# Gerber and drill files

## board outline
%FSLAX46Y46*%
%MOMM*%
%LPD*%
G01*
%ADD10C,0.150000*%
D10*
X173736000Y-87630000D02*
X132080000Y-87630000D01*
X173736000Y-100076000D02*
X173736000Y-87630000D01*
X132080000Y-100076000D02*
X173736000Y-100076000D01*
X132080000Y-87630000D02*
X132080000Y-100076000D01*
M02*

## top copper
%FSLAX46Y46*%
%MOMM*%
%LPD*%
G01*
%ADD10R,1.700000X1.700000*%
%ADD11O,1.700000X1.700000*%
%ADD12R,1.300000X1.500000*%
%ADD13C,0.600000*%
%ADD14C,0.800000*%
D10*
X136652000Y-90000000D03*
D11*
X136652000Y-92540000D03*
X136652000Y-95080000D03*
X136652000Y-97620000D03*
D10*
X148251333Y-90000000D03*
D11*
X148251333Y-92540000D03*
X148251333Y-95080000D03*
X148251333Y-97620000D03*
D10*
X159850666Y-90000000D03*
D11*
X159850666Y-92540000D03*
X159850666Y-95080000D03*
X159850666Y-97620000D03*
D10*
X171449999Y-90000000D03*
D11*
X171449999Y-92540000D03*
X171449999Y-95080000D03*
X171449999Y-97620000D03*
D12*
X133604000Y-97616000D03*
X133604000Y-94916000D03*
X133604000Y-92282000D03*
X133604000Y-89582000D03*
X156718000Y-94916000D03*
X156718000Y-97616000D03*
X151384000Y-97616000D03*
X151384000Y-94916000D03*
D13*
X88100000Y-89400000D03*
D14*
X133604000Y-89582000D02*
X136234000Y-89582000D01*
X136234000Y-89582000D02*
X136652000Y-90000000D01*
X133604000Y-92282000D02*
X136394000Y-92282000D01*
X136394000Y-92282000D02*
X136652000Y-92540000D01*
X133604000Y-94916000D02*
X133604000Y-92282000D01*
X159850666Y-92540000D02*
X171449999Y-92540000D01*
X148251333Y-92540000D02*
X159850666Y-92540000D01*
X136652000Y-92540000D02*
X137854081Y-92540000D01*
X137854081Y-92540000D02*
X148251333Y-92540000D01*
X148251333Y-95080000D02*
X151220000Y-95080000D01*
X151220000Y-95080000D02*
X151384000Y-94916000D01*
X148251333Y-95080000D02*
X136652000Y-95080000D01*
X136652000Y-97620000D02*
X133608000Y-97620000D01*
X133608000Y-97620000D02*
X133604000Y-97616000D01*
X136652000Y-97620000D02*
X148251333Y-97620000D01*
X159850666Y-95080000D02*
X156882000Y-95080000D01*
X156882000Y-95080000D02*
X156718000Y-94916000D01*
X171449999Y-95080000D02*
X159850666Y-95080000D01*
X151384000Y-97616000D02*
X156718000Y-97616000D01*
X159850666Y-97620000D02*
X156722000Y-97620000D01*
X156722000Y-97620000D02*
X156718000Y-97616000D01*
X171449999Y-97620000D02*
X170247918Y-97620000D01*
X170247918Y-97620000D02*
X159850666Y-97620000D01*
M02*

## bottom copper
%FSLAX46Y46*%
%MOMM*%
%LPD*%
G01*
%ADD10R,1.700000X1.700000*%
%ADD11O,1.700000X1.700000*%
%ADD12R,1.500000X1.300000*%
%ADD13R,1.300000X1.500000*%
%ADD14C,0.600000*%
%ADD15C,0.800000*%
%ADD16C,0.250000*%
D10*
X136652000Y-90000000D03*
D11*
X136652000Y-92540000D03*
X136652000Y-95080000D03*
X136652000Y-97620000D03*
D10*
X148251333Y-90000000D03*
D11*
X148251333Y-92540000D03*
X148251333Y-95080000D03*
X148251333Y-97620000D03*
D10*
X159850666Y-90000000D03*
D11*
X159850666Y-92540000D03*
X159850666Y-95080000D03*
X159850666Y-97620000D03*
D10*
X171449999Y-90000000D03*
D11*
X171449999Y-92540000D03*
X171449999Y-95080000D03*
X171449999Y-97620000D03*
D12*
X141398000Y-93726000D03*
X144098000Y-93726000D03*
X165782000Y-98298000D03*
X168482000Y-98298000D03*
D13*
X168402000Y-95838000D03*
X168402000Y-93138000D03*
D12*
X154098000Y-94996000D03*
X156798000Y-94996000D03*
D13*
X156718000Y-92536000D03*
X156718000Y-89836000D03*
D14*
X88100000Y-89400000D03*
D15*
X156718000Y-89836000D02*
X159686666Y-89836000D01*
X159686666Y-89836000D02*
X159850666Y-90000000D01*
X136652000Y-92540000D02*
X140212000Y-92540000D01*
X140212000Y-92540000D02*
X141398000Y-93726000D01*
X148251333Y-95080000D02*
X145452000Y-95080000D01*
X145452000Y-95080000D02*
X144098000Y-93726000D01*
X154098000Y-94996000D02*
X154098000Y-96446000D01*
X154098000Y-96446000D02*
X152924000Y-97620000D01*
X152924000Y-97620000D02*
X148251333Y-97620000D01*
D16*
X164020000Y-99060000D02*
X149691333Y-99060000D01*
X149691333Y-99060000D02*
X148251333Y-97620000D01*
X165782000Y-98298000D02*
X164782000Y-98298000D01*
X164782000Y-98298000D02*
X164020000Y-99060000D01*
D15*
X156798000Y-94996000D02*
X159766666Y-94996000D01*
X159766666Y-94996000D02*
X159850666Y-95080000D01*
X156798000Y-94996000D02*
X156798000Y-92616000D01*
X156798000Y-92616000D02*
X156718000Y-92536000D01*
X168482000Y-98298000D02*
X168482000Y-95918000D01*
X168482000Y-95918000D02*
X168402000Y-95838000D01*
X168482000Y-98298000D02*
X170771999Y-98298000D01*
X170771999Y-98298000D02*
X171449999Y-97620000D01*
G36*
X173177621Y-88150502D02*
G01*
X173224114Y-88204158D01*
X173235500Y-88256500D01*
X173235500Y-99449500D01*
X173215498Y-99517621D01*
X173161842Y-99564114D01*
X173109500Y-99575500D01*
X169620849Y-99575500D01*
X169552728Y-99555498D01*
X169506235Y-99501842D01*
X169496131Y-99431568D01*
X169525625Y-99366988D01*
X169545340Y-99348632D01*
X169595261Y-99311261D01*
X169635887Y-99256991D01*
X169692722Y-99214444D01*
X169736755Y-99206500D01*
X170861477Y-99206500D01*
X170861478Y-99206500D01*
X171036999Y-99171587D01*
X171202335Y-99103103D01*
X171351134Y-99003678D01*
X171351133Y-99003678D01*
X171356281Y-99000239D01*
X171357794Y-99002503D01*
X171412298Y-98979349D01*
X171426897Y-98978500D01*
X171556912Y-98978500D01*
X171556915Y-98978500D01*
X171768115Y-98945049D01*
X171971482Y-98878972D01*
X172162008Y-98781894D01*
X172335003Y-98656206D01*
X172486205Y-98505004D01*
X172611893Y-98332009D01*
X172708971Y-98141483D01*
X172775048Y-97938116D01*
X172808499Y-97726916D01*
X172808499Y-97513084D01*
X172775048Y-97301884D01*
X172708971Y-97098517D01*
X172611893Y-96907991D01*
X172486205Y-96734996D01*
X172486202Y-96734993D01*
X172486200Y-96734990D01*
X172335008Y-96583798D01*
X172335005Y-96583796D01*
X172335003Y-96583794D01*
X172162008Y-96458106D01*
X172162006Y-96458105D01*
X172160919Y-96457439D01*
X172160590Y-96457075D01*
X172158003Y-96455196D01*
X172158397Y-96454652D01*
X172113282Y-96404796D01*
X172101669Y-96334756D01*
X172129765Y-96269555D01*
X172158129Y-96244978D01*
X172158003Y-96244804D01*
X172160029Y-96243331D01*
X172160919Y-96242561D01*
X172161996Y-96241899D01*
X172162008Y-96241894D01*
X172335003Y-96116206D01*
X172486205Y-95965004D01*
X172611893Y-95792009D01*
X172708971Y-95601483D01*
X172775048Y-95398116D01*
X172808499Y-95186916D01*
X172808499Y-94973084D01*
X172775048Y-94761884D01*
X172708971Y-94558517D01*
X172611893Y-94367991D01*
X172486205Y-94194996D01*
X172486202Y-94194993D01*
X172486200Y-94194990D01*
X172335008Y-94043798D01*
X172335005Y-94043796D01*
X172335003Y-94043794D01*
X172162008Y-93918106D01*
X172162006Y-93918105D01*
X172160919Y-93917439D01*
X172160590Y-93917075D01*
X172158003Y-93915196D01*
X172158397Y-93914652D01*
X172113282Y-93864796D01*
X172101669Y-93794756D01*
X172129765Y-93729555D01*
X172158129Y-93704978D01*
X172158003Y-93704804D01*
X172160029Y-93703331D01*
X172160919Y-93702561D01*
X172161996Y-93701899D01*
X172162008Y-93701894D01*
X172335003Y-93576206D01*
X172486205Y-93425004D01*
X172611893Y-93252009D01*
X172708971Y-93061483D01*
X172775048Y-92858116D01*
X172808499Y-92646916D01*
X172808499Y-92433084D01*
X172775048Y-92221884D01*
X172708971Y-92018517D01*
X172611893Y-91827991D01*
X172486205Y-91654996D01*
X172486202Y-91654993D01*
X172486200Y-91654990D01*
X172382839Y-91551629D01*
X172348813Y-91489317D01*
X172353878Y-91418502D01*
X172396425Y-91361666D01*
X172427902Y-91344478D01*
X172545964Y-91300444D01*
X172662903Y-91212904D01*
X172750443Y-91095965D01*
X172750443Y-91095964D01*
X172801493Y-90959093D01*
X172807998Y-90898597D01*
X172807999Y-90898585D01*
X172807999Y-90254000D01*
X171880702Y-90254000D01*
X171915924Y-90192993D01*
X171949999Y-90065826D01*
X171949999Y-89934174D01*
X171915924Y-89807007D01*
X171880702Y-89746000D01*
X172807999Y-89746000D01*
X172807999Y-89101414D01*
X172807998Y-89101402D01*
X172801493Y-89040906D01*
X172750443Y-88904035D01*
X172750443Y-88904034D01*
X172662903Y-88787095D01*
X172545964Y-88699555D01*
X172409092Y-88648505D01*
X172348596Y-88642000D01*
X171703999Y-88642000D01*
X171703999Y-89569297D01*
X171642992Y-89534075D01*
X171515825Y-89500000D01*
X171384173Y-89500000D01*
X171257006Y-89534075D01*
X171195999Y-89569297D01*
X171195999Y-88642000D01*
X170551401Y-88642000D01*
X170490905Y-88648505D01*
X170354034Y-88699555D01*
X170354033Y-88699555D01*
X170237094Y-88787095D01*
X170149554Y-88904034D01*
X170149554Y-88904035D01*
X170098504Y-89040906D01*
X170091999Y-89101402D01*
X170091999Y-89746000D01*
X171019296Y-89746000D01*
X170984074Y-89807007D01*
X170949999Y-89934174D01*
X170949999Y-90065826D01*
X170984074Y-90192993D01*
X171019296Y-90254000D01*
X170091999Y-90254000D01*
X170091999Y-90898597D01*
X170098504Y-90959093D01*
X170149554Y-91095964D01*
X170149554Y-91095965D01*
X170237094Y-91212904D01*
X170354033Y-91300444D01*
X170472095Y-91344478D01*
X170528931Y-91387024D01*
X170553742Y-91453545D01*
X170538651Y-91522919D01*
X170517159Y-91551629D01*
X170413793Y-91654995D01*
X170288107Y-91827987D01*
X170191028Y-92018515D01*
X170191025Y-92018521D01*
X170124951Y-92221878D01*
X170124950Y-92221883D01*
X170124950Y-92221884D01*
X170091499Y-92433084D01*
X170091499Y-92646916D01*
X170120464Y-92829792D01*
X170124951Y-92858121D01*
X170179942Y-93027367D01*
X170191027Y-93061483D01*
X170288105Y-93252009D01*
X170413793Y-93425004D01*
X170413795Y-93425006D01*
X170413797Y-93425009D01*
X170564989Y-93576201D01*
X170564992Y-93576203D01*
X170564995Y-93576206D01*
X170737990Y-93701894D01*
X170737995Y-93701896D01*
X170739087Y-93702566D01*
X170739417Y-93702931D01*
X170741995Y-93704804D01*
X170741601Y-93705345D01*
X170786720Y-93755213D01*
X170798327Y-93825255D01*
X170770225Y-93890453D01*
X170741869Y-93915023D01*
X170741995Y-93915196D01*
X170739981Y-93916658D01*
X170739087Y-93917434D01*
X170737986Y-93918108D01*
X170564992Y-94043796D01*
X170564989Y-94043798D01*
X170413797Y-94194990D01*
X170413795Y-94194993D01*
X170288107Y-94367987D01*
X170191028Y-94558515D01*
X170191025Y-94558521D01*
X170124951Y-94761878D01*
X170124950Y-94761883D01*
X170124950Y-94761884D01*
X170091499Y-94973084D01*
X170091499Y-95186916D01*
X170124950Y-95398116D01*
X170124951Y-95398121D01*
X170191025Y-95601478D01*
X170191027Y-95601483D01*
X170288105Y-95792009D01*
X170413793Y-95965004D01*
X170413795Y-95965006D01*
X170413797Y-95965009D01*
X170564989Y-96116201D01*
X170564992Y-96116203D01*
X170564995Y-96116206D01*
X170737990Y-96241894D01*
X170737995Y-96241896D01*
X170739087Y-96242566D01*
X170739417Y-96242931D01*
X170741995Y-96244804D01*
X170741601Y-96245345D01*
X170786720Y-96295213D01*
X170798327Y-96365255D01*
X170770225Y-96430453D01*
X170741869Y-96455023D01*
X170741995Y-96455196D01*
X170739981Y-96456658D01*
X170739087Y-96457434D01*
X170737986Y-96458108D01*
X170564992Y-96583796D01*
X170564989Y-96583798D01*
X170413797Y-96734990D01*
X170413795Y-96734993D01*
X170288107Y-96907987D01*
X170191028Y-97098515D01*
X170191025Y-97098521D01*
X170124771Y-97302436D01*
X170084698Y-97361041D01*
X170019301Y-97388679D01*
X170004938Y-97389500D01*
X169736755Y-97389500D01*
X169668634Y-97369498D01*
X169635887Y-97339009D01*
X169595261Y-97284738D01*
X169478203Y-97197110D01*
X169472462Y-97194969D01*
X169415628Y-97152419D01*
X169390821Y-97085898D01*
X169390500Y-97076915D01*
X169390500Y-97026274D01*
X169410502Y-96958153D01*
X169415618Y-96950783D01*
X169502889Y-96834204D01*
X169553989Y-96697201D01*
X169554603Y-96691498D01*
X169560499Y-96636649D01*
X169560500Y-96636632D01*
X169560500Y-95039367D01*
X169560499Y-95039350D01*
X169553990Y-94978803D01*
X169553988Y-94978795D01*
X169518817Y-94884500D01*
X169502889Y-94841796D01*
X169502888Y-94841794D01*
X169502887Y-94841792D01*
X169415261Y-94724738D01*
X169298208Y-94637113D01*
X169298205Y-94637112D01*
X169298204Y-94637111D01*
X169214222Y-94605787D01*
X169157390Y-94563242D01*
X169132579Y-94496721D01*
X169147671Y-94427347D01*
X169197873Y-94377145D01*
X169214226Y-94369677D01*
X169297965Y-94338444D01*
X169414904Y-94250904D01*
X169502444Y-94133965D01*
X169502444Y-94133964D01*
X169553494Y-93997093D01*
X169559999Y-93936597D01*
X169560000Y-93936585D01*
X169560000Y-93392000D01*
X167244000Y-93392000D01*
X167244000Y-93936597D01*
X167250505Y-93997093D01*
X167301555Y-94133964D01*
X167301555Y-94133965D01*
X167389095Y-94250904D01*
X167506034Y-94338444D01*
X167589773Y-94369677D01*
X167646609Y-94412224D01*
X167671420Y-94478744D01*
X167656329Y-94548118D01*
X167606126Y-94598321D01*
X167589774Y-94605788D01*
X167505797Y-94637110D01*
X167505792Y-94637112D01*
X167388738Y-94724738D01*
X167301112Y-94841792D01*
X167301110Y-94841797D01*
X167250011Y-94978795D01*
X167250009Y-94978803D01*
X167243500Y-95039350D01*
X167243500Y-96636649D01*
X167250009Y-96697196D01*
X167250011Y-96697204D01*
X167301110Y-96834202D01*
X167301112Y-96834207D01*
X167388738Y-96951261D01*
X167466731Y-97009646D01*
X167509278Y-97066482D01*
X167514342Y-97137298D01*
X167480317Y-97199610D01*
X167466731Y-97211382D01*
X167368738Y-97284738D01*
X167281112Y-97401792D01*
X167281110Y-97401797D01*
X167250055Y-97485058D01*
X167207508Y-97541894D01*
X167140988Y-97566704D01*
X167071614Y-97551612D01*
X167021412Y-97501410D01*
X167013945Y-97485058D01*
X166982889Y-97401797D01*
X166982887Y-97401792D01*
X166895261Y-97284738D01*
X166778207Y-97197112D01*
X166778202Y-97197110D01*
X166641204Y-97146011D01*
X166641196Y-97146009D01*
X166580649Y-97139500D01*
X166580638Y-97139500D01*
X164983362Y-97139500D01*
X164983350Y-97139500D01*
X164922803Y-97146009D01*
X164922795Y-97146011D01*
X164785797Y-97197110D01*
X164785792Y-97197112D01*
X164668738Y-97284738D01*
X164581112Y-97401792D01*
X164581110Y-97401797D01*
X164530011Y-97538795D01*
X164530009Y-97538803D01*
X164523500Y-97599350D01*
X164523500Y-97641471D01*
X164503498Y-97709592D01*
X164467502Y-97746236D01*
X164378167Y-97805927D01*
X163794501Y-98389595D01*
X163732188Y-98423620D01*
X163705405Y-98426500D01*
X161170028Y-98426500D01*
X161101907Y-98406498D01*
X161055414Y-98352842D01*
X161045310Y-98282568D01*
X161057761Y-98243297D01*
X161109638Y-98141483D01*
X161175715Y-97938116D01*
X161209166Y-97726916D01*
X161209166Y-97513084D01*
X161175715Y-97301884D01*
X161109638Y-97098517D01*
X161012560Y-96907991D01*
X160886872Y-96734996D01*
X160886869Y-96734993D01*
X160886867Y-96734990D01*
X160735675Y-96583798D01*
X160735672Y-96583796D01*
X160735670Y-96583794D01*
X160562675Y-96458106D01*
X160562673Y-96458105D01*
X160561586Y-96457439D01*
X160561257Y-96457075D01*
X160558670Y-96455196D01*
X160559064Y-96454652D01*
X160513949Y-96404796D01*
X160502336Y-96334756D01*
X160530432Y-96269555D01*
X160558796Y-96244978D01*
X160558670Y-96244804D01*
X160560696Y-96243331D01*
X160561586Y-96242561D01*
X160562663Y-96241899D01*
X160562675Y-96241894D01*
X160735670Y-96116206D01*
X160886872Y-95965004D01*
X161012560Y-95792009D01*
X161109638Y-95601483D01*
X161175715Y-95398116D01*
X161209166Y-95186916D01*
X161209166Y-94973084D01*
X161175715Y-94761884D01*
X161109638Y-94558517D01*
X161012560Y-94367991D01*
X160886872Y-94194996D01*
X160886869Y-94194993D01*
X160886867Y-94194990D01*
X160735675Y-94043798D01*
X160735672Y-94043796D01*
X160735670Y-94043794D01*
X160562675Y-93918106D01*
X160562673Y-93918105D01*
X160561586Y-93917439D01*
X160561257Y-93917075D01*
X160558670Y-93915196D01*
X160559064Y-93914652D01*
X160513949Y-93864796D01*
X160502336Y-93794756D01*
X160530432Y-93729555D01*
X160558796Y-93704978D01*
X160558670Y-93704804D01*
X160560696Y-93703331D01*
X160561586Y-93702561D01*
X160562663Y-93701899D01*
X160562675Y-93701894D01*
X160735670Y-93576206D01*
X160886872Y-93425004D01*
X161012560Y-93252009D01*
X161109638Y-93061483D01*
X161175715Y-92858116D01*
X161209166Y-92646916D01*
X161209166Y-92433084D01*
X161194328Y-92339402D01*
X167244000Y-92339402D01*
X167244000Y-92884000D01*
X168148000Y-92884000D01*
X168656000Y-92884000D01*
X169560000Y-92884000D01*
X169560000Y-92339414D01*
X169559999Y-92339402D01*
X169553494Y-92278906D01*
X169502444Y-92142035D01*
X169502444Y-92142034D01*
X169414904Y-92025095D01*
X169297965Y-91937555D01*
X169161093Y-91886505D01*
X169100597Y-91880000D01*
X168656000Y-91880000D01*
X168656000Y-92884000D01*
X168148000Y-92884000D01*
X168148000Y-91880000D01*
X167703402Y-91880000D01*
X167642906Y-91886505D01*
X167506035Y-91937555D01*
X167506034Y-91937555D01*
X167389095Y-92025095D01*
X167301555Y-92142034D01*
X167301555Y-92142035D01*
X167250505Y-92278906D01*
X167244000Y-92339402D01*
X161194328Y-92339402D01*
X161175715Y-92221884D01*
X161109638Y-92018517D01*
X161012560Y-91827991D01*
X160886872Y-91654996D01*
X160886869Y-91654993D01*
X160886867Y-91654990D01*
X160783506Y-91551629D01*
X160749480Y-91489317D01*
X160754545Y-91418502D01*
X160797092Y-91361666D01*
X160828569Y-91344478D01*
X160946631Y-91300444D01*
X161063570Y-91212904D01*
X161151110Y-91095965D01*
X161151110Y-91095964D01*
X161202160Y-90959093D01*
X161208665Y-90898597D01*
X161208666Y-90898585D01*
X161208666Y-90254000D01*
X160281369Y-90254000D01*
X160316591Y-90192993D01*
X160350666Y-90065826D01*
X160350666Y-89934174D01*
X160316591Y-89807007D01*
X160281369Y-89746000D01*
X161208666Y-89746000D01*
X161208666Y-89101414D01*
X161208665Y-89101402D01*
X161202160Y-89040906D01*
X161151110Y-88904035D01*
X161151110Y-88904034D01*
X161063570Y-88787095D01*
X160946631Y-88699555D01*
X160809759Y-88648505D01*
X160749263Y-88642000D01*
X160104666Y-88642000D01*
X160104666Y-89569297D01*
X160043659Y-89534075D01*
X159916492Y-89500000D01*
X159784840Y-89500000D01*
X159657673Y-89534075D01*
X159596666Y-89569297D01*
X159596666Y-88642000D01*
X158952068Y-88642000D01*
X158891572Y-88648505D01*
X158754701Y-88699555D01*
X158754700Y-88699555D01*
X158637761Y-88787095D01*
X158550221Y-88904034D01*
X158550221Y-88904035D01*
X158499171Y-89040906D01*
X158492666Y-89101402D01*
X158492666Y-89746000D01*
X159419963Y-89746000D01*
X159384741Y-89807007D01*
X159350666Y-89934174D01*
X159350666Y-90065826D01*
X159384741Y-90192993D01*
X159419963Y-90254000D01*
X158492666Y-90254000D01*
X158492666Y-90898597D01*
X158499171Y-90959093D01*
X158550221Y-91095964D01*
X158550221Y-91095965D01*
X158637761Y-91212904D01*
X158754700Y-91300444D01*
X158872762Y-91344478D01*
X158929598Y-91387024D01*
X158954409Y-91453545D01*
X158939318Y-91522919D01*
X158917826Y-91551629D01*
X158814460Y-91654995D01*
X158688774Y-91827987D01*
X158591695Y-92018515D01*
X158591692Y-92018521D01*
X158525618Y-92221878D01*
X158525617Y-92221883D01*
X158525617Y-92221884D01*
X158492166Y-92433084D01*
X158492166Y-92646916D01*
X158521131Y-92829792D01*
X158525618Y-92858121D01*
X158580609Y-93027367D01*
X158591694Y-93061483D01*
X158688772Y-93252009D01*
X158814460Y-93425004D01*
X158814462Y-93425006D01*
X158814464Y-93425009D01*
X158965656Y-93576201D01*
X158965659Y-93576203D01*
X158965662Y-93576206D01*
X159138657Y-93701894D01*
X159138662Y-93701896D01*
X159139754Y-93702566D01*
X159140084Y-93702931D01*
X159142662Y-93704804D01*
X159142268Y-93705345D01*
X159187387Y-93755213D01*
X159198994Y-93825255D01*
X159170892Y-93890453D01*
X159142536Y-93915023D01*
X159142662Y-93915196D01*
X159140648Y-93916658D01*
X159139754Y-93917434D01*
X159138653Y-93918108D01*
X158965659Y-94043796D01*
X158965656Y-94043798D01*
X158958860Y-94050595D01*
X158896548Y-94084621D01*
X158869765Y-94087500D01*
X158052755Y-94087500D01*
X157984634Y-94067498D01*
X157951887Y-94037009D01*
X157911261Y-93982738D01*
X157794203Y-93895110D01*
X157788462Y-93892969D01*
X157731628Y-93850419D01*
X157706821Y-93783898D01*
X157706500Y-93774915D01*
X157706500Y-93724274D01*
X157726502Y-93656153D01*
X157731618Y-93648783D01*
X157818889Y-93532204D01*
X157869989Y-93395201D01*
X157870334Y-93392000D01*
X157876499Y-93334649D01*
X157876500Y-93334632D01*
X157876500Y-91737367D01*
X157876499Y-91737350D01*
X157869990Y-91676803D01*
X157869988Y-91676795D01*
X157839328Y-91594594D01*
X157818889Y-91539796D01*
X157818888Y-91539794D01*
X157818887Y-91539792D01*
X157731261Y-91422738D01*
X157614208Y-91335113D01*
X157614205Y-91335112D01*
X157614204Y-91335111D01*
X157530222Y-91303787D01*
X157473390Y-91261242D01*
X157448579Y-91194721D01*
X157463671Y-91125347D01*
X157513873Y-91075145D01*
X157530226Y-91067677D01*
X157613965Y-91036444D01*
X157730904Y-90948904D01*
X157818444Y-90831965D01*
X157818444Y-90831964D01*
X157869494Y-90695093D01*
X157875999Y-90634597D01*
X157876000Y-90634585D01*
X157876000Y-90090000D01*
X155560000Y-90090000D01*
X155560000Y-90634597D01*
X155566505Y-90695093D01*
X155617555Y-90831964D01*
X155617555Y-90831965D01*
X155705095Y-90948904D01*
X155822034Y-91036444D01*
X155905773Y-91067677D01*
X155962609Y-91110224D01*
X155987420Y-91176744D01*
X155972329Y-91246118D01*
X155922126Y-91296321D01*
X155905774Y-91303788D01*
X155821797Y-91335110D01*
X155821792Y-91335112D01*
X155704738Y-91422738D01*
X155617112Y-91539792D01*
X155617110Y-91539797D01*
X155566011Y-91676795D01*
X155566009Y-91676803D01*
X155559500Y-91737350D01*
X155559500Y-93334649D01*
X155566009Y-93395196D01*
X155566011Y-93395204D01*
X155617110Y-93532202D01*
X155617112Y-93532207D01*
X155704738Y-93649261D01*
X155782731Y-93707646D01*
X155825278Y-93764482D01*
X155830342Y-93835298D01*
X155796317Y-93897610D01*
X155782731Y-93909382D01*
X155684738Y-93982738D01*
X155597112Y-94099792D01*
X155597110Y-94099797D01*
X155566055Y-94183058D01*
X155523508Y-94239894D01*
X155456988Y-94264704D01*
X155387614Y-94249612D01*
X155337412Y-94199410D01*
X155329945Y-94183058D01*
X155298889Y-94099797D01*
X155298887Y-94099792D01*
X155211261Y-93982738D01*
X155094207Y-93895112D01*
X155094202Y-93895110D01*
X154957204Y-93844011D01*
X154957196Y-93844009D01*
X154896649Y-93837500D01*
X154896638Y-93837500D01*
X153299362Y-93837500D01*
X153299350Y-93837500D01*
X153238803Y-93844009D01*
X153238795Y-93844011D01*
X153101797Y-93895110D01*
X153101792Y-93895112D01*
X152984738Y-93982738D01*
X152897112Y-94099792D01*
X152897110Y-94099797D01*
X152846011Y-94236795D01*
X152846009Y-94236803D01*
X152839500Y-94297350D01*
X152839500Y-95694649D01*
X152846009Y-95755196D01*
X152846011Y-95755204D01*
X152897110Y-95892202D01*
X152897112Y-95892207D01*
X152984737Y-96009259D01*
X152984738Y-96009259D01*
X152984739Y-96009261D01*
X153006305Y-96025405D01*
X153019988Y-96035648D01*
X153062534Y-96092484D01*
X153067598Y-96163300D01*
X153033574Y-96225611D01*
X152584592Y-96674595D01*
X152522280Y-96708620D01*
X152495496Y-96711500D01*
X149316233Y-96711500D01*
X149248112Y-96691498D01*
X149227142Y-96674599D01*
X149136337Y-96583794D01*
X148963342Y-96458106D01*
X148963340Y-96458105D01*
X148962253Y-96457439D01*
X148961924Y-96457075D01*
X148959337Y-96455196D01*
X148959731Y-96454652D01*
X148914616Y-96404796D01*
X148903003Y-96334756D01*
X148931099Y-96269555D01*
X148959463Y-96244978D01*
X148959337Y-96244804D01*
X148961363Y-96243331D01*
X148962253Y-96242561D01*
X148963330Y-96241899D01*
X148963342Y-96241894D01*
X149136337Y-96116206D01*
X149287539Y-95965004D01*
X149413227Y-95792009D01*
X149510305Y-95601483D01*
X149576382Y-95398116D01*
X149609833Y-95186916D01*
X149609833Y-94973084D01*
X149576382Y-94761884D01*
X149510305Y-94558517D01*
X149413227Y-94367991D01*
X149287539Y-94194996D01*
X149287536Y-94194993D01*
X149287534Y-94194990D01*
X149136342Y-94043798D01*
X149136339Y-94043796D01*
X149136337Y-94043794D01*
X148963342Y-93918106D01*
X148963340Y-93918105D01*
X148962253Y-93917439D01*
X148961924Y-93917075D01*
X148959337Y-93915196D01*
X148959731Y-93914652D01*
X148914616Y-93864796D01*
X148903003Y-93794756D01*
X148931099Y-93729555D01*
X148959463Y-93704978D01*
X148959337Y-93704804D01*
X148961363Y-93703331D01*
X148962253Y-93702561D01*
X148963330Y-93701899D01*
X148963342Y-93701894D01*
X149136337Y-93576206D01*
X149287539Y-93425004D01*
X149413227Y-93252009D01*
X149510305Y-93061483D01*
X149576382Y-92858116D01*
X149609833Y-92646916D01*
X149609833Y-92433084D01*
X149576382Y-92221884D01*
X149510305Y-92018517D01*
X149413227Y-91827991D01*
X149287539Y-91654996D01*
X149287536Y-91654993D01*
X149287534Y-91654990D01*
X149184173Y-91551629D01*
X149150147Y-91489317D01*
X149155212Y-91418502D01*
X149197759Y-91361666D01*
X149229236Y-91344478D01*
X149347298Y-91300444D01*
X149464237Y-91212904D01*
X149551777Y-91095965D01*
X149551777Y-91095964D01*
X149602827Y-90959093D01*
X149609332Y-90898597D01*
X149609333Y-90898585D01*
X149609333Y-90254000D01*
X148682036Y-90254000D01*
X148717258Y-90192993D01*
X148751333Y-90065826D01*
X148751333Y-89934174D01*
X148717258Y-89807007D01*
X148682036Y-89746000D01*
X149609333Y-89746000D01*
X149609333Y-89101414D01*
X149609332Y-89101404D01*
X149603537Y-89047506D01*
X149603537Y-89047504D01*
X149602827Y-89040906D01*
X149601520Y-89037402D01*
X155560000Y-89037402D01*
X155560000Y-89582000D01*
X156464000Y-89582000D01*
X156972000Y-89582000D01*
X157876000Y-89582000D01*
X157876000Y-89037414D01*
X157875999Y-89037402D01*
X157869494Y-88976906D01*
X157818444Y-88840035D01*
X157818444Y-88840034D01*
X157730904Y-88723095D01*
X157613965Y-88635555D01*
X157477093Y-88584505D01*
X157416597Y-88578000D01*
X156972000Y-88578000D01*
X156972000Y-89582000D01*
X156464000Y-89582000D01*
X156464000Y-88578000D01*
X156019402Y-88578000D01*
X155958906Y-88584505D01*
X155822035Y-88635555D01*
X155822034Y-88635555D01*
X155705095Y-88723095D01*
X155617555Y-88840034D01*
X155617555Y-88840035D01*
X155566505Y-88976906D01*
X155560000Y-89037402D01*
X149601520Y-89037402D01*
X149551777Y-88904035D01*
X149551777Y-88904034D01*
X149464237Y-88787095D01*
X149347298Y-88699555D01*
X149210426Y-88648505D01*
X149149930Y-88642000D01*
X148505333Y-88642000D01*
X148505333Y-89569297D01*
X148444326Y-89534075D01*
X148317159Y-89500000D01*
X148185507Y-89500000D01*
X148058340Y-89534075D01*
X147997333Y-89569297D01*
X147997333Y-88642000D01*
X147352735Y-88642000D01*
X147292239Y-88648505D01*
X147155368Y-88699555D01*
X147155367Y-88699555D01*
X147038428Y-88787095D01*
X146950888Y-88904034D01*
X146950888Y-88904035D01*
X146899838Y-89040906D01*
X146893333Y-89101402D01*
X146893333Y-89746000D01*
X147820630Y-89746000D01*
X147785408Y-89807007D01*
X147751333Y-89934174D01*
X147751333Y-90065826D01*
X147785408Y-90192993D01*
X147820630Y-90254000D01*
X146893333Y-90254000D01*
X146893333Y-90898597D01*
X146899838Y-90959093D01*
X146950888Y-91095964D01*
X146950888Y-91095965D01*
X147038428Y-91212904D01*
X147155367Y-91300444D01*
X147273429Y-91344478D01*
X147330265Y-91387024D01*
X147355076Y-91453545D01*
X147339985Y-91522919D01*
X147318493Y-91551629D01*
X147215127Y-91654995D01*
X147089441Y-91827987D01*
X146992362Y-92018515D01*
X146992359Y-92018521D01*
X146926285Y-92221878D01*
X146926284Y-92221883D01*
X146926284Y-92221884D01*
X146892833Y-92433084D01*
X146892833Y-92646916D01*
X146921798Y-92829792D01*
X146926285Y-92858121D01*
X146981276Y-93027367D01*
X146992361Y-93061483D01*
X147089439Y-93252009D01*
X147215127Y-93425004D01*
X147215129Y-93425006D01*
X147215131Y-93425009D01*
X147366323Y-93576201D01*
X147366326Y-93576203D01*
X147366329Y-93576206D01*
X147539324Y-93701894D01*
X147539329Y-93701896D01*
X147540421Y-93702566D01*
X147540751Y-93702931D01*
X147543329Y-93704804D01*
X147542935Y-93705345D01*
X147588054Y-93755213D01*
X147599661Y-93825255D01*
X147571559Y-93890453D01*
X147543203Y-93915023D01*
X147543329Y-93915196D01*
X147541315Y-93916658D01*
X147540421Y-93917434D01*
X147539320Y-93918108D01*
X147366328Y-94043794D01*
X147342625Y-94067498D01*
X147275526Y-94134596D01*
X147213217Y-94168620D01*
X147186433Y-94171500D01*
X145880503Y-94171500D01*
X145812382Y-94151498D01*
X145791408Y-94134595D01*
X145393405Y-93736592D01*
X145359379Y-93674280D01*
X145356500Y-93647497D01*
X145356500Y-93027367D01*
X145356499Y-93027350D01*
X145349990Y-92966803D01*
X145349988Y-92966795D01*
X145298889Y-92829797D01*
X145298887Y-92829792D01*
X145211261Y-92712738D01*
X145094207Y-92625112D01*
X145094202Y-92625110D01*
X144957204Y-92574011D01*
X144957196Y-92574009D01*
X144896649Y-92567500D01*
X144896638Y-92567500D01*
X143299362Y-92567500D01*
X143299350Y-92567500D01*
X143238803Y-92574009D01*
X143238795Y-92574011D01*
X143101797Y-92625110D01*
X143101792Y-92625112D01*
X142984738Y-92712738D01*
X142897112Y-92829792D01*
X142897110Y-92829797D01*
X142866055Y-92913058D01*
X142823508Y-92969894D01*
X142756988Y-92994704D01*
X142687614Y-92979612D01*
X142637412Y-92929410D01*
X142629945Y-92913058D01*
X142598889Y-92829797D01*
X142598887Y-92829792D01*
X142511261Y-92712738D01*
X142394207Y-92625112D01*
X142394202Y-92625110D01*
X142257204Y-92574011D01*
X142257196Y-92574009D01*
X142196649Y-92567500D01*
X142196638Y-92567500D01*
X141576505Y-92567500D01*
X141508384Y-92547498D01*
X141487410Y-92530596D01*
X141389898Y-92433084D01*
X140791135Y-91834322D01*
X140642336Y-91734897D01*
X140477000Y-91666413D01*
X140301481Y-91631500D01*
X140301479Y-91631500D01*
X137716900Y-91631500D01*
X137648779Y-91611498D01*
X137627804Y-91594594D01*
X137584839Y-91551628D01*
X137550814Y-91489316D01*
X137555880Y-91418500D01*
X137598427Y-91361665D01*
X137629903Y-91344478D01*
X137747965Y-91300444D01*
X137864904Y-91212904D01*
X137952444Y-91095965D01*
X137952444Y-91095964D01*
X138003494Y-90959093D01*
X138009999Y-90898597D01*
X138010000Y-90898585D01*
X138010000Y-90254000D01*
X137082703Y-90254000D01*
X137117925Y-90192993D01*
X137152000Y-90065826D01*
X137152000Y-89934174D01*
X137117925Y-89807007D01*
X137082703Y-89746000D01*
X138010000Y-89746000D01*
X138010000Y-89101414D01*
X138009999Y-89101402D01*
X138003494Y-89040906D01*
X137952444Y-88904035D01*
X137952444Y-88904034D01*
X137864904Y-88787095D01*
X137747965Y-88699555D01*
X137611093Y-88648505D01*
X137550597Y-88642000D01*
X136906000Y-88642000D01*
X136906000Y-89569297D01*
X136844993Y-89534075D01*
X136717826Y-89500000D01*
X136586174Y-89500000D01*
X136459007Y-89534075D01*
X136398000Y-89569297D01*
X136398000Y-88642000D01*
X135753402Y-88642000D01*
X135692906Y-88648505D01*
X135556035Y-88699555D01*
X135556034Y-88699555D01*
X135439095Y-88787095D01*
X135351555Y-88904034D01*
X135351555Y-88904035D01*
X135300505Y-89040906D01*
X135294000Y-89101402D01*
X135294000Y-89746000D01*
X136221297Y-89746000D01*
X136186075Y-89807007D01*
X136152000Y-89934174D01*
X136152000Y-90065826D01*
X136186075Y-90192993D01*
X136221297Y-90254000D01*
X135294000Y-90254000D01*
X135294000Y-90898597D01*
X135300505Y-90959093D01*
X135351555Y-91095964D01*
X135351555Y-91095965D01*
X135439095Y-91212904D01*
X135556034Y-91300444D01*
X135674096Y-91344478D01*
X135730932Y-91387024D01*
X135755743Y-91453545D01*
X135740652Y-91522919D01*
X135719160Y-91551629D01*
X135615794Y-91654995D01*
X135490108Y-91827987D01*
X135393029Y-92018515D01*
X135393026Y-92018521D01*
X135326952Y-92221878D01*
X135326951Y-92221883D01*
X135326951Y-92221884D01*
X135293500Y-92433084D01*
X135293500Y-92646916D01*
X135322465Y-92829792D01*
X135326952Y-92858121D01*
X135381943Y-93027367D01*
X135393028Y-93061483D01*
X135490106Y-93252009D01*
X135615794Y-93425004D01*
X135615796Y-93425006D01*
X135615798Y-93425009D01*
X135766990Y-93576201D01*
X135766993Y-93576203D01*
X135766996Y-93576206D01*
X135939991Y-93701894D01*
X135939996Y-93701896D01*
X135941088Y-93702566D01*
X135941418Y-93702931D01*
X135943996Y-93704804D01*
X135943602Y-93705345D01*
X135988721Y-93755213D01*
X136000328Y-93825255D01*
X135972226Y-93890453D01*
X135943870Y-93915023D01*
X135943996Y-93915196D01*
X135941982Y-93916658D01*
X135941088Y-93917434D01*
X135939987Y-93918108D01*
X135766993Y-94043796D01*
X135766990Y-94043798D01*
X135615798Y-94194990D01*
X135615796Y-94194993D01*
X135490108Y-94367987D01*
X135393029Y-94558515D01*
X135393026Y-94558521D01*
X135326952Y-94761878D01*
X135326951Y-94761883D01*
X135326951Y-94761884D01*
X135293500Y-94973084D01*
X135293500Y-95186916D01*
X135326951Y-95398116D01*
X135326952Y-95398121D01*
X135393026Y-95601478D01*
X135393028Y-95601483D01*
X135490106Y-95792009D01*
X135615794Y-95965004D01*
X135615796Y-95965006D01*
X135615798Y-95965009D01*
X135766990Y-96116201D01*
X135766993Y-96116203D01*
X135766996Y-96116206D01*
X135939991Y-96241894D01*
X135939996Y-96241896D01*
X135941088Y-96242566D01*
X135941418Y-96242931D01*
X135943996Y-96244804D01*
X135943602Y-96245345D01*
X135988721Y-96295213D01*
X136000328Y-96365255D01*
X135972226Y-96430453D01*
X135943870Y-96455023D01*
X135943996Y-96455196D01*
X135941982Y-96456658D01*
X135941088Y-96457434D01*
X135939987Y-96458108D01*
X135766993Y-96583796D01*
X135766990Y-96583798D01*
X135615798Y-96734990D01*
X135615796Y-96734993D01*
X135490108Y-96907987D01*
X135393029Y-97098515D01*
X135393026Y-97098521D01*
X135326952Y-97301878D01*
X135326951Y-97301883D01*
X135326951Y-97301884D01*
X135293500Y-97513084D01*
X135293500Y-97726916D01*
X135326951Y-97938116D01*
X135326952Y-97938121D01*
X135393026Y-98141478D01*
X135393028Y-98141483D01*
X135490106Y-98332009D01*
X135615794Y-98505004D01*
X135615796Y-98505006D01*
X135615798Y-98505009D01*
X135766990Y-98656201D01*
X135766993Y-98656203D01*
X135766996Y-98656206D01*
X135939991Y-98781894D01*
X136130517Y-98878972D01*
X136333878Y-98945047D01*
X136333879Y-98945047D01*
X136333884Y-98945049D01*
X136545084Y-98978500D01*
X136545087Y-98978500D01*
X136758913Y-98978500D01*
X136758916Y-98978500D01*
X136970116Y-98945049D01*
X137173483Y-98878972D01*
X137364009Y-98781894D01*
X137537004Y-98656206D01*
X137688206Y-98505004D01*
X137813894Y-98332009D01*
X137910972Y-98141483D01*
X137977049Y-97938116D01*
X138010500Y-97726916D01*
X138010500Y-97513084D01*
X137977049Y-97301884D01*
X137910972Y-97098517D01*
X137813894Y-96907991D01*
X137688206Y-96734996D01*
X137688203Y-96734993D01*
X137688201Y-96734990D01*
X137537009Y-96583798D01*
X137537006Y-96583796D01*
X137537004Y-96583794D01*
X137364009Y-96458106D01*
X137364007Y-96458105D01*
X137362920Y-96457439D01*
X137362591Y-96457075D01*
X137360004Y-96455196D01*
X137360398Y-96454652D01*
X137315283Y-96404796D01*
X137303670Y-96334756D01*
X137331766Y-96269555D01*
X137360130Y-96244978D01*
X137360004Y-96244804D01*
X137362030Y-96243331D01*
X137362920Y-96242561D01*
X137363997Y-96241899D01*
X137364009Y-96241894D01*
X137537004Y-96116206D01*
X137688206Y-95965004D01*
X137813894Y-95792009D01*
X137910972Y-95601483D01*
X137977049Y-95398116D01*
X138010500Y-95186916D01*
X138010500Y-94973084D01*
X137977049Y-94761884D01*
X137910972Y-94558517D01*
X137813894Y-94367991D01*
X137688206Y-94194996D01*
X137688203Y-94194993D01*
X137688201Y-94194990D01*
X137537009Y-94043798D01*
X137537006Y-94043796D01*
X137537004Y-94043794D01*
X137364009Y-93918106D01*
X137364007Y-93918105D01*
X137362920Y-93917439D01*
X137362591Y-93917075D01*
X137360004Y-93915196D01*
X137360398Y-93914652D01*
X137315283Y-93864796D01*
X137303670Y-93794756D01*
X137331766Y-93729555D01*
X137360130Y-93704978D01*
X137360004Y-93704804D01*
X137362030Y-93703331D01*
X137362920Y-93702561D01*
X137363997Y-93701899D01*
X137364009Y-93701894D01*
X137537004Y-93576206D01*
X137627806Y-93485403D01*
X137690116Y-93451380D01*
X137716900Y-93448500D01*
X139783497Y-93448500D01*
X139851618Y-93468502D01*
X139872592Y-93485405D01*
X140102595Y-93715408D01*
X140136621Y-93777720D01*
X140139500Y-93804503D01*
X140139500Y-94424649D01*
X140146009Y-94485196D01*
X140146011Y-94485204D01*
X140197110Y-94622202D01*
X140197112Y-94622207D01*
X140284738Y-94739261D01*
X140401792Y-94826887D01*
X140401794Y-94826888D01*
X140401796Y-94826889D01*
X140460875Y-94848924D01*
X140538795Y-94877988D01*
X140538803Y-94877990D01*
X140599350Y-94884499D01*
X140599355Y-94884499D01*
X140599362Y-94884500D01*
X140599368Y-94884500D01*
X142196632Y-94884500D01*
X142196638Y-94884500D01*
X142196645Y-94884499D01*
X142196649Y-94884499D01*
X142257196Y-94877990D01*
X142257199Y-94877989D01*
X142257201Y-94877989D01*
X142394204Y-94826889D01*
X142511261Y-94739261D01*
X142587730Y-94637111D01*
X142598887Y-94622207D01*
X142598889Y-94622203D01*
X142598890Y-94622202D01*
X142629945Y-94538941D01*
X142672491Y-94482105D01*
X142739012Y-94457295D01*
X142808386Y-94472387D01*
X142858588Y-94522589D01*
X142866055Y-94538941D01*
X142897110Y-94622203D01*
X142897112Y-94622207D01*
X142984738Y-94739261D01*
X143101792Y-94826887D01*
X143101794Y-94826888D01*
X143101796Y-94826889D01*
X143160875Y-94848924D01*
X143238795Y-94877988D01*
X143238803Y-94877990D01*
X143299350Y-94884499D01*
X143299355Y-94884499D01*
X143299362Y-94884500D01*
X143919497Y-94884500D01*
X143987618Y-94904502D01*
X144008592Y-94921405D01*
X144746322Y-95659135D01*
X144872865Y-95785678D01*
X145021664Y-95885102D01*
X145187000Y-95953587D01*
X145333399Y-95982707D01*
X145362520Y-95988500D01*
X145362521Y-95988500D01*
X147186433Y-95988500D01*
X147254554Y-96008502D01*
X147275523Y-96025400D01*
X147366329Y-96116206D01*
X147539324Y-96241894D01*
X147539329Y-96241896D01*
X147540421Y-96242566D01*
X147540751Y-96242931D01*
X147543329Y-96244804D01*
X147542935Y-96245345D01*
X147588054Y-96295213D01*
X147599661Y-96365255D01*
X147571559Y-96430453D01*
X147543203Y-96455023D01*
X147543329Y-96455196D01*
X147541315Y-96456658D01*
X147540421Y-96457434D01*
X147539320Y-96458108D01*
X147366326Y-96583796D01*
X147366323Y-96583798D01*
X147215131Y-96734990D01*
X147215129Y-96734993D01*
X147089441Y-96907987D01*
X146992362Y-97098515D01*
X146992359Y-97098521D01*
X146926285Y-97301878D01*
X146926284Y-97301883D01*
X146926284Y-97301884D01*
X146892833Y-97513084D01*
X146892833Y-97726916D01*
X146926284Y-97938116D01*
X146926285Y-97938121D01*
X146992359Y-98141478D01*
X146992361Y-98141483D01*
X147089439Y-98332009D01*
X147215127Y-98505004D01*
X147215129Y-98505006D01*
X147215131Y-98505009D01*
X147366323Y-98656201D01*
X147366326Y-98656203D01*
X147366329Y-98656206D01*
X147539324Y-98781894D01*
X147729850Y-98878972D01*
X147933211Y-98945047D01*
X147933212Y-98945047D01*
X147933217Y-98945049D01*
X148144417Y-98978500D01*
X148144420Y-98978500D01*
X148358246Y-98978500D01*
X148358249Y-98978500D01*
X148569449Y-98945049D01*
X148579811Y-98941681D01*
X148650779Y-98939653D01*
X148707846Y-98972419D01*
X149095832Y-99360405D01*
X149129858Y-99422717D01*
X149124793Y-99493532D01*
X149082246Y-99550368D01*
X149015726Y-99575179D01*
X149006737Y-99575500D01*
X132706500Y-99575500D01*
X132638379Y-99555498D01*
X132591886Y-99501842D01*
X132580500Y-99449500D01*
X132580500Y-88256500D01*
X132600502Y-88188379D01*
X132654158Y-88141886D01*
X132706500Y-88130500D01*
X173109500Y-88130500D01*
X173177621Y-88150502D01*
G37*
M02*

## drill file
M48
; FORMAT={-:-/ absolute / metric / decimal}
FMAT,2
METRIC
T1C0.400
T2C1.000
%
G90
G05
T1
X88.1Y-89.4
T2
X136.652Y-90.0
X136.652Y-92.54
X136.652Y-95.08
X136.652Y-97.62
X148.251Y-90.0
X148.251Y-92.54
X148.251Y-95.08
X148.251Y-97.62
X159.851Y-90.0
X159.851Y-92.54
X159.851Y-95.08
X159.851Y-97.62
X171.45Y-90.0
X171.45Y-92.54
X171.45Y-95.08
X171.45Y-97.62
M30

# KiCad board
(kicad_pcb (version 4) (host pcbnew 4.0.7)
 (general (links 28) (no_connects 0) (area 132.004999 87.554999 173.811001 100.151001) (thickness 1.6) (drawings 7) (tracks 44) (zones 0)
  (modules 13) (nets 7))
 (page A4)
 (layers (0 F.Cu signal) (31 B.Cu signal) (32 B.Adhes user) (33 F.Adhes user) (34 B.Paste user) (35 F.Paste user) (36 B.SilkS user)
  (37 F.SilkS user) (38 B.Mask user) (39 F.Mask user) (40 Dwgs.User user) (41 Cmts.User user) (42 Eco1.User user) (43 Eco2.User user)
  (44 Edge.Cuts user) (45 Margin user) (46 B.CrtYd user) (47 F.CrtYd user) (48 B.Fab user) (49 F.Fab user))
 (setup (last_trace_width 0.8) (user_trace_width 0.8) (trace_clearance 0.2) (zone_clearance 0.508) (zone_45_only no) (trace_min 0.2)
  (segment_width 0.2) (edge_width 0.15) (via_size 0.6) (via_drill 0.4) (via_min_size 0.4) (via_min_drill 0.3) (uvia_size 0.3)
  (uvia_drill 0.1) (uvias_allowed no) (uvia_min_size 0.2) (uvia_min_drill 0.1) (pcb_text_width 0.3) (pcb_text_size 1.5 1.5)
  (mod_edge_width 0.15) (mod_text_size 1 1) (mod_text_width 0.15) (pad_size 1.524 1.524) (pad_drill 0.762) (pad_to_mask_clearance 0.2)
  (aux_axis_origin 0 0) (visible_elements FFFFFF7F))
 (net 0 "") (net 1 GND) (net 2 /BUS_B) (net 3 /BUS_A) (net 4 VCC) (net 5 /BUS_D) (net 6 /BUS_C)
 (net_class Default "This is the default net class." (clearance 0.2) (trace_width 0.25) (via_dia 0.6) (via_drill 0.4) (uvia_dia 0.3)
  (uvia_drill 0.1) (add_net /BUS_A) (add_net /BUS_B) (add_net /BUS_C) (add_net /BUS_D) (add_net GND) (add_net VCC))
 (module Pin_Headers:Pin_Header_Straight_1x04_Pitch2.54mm (layer F.Cu) (at 136.652 90)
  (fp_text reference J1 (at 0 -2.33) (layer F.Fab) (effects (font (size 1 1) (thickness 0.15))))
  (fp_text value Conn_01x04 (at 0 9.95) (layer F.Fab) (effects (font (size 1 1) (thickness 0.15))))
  (pad 1 thru_hole rect (at 0 0) (size 1.7 1.7) (drill 1) (layers *.Cu *.Mask) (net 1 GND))
  (pad 2 thru_hole oval (at 0 2.54) (size 1.7 1.7) (drill 1) (layers *.Cu *.Mask) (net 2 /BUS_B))
  (pad 3 thru_hole oval (at 0 5.08) (size 1.7 1.7) (drill 1) (layers *.Cu *.Mask) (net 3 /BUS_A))
  (pad 4 thru_hole oval (at 0 7.62) (size 1.7 1.7) (drill 1) (layers *.Cu *.Mask) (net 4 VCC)))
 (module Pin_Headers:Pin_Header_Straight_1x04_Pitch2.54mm (layer F.Cu) (at 148.251333 90)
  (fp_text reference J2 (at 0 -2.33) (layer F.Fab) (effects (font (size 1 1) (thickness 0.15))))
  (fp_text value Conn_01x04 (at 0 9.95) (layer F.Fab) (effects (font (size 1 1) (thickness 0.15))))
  (pad 1 thru_hole rect (at 0 0) (size 1.7 1.7) (drill 1) (layers *.Cu *.Mask) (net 1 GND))
  (pad 2 thru_hole oval (at 0 2.54) (size 1.7 1.7) (drill 1) (layers *.Cu *.Mask) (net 2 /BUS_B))
  (pad 3 thru_hole oval (at 0 5.08) (size 1.7 1.7) (drill 1) (layers *.Cu *.Mask) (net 3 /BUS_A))
  (pad 4 thru_hole oval (at 0 7.62) (size 1.7 1.7) (drill 1) (layers *.Cu *.Mask) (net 4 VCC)))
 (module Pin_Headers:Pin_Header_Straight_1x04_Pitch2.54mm (layer F.Cu) (at 159.850666 90)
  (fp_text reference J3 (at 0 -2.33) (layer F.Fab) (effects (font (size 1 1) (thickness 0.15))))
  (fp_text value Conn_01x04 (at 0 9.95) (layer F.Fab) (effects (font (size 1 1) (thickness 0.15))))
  (pad 1 thru_hole rect (at 0 0) (size 1.7 1.7) (drill 1) (layers *.Cu *.Mask) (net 1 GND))
  (pad 2 thru_hole oval (at 0 2.54) (size 1.7 1.7) (drill 1) (layers *.Cu *.Mask) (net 2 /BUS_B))
  (pad 3 thru_hole oval (at 0 5.08) (size 1.7 1.7) (drill 1) (layers *.Cu *.Mask) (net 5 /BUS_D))
  (pad 4 thru_hole oval (at 0 7.62) (size 1.7 1.7) (drill 1) (layers *.Cu *.Mask) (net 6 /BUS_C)))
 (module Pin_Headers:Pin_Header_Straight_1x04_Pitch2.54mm (layer F.Cu) (at 171.449999 90)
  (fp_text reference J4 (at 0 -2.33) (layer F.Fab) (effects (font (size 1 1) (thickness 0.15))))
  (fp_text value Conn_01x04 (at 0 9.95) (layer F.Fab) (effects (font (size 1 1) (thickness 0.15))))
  (pad 1 thru_hole rect (at 0 0) (size 1.7 1.7) (drill 1) (layers *.Cu *.Mask) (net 1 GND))
  (pad 2 thru_hole oval (at 0 2.54) (size 1.7 1.7) (drill 1) (layers *.Cu *.Mask) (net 2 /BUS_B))
  (pad 3 thru_hole oval (at 0 5.08) (size 1.7 1.7) (drill 1) (layers *.Cu *.Mask) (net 5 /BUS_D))
  (pad 4 thru_hole oval (at 0 7.62) (size 1.7 1.7) (drill 1) (layers *.Cu *.Mask) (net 6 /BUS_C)))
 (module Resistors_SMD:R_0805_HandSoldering (layer F.Cu) (at 133.604 96.266 90)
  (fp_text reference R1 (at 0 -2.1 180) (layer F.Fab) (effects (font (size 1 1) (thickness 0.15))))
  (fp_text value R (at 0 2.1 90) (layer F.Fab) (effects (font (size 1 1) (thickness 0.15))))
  (pad 1 smd rect (at -1.35 0 90) (size 1.5 1.3) (layers F.Cu F.Paste F.Mask) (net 4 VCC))
  (pad 2 smd rect (at 1.35 0 90) (size 1.5 1.3) (layers F.Cu F.Paste F.Mask) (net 2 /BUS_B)))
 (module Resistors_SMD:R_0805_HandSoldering (layer F.Cu) (at 133.604 90.932 90)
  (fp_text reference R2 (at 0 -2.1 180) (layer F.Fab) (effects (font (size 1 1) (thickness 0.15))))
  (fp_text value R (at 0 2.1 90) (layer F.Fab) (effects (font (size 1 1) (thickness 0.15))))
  (pad 1 smd rect (at -1.35 0 90) (size 1.5 1.3) (layers F.Cu F.Paste F.Mask) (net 2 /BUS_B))
  (pad 2 smd rect (at 1.35 0 90) (size 1.5 1.3) (layers F.Cu F.Paste F.Mask) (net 1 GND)))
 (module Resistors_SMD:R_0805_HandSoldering (layer B.Cu) (at 142.748 93.726)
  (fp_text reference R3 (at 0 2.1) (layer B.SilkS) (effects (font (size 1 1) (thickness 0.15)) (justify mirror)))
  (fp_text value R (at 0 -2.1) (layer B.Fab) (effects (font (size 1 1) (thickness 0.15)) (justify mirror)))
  (pad 1 smd rect (at -1.35 0) (size 1.5 1.3) (layers B.Cu B.Paste B.Mask) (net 2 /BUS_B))
  (pad 2 smd rect (at 1.35 0) (size 1.5 1.3) (layers B.Cu B.Paste B.Mask) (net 3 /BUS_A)))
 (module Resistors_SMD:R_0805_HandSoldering (layer F.Cu) (at 156.718 96.266 270)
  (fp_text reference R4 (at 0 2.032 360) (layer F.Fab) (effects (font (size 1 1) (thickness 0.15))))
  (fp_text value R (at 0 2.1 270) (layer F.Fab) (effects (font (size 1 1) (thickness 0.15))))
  (pad 1 smd rect (at -1.35 0 270) (size 1.5 1.3) (layers F.Cu F.Paste F.Mask) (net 5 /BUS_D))
  (pad 2 smd rect (at 1.35 0 270) (size 1.5 1.3) (layers F.Cu F.Paste F.Mask) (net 6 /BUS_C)))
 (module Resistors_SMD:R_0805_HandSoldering (layer B.Cu) (at 167.132 98.298)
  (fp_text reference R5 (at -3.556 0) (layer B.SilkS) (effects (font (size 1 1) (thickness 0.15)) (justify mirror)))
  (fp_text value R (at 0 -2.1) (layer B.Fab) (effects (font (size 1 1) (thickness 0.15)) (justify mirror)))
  (pad 1 smd rect (at -1.35 0) (size 1.5 1.3) (layers B.Cu B.Paste B.Mask) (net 4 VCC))
  (pad 2 smd rect (at 1.35 0) (size 1.5 1.3) (layers B.Cu B.Paste B.Mask) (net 6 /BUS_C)))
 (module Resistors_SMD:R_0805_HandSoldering (layer B.Cu) (at 168.402 94.488 90)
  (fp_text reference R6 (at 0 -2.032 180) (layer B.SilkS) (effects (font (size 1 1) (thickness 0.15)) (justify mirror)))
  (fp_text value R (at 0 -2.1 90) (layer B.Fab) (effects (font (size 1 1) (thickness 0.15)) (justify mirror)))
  (pad 1 smd rect (at -1.35 0 90) (size 1.5 1.3) (layers B.Cu B.Paste B.Mask) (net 6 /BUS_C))
  (pad 2 smd rect (at 1.35 0 90) (size 1.5 1.3) (layers B.Cu B.Paste B.Mask) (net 1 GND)))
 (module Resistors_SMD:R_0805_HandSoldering (layer B.Cu) (at 155.448 94.996)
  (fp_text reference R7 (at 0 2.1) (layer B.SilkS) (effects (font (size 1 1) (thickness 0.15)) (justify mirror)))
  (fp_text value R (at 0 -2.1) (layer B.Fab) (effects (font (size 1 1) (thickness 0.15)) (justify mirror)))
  (pad 1 smd rect (at -1.35 0) (size 1.5 1.3) (layers B.Cu B.Paste B.Mask) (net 4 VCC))
  (pad 2 smd rect (at 1.35 0) (size 1.5 1.3) (layers B.Cu B.Paste B.Mask) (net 5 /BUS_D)))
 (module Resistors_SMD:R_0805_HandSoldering (layer B.Cu) (at 156.718 91.186 90)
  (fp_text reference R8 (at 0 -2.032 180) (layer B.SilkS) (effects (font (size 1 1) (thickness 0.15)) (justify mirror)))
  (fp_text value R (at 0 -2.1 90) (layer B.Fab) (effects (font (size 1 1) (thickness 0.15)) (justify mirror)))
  (pad 1 smd rect (at -1.35 0 90) (size 1.5 1.3) (layers B.Cu B.Paste B.Mask) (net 5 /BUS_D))
  (pad 2 smd rect (at 1.35 0 90) (size 1.5 1.3) (layers B.Cu B.Paste B.Mask) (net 1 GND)))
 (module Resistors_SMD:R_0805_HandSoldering (layer F.Cu) (at 151.384 96.266 90)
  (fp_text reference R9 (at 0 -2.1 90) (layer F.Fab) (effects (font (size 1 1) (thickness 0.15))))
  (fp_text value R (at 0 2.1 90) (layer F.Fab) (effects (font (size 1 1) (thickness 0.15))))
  (pad 1 smd rect (at -1.35 0 90) (size 1.5 1.3) (layers F.Cu F.Paste F.Mask) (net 6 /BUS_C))
  (pad 2 smd rect (at 1.35 0 90) (size 1.5 1.3) (layers F.Cu F.Paste F.Mask) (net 3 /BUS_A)))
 (gr_line (start 173.736 87.63) (end 132.08 87.63) (layer Edge.Cuts) (width 0.15))
 (gr_line (start 173.736 100.076) (end 173.736 87.63) (layer Edge.Cuts) (width 0.15))
 (gr_line (start 132.08 100.076) (end 173.736 100.076) (layer Edge.Cuts) (width 0.15))
 (gr_line (start 132.08 87.63) (end 132.08 100.076) (layer Edge.Cuts) (width 0.15))
 (via (at 88.1 89.4) (size 0.6) (drill 0.4) (layers F.Cu B.Cu) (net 1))
 (segment (start 156.718 89.836) (end 159.686666 89.836) (width 0.8) (layer B.Cu) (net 1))
 (segment (start 159.686666 89.836) (end 159.850666 90) (width 0.8) (layer B.Cu) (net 1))
 (segment (start 133.604 89.582) (end 136.234 89.582) (width 0.8) (layer F.Cu) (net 1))
 (segment (start 136.234 89.582) (end 136.652 90) (width 0.8) (layer F.Cu) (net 1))
 (segment (start 136.652 92.54) (end 140.212 92.54) (width 0.8) (layer B.Cu) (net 2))
 (segment (start 140.212 92.54) (end 141.398 93.726) (width 0.8) (layer B.Cu) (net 2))
 (segment (start 133.604 92.282) (end 136.394 92.282) (width 0.8) (layer F.Cu) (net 2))
 (segment (start 136.394 92.282) (end 136.652 92.54) (width 0.8) (layer F.Cu) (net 2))
 (segment (start 133.604 94.916) (end 133.604 92.282) (width 0.8) (layer F.Cu) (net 2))
 (segment (start 159.850666 92.54) (end 171.449999 92.54) (width 0.8) (layer F.Cu) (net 2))
 (segment (start 148.251333 92.54) (end 159.850666 92.54) (width 0.8) (layer F.Cu) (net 2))
 (segment (start 136.652 92.54) (end 137.854081 92.54) (width 0.8) (layer F.Cu) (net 2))
 (segment (start 137.854081 92.54) (end 148.251333 92.54) (width 0.8) (layer F.Cu) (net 2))
 (segment (start 148.251333 95.08) (end 151.22 95.08) (width 0.8) (layer F.Cu) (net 3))
 (segment (start 151.22 95.08) (end 151.384 94.916) (width 0.8) (layer F.Cu) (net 3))
 (segment (start 148.251333 95.08) (end 145.452 95.08) (width 0.8) (layer B.Cu) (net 3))
 (segment (start 145.452 95.08) (end 144.098 93.726) (width 0.8) (layer B.Cu) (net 3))
 (segment (start 148.251333 95.08) (end 136.652 95.08) (width 0.8) (layer F.Cu) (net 3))
 (segment (start 154.098 94.996) (end 154.098 96.446) (width 0.8) (layer B.Cu) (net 4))
 (segment (start 154.098 96.446) (end 152.924 97.62) (width 0.8) (layer B.Cu) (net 4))
 (segment (start 152.924 97.62) (end 148.251333 97.62) (width 0.8) (layer B.Cu) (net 4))
 (segment (start 164.02 99.06) (end 149.691333 99.06) (width 0.25) (layer B.Cu) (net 4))
 (segment (start 149.691333 99.06) (end 148.251333 97.62) (width 0.25) (layer B.Cu) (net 4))
 (segment (start 165.782 98.298) (end 164.782 98.298) (width 0.25) (layer B.Cu) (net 4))
 (segment (start 164.782 98.298) (end 164.02 99.06) (width 0.25) (layer B.Cu) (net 4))
 (segment (start 136.652 97.62) (end 133.608 97.62) (width 0.8) (layer F.Cu) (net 4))
 (segment (start 133.608 97.62) (end 133.604 97.616) (width 0.8) (layer F.Cu) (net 4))
 (segment (start 136.652 97.62) (end 148.251333 97.62) (width 0.8) (layer F.Cu) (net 4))
 (segment (start 156.798 94.996) (end 159.766666 94.996) (width 0.8) (layer B.Cu) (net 5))
 (segment (start 159.766666 94.996) (end 159.850666 95.08) (width 0.8) (layer B.Cu) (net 5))
 (segment (start 156.798 94.996) (end 156.798 92.616) (width 0.8) (layer B.Cu) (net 5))
 (segment (start 156.798 92.616) (end 156.718 92.536) (width 0.8) (layer B.Cu) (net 5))
 (segment (start 159.850666 95.08) (end 156.882 95.08) (width 0.8) (layer F.Cu) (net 5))
 (segment (start 156.882 95.08) (end 156.718 94.916) (width 0.8) (layer F.Cu) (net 5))
 (segment (start 171.449999 95.08) (end 159.850666 95.08) (width 0.8) (layer F.Cu) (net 5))
 (segment (start 151.384 97.616) (end 156.718 97.616) (width 0.8) (layer F.Cu) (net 6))
 (segment (start 168.482 98.298) (end 168.482 95.918) (width 0.8) (layer B.Cu) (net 6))
 (segment (start 168.482 95.918) (end 168.402 95.838) (width 0.8) (layer B.Cu) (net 6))
 (segment (start 168.482 98.298) (end 170.771999 98.298) (width 0.8) (layer B.Cu) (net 6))
 (segment (start 170.771999 98.298) (end 171.449999 97.62) (width 0.8) (layer B.Cu) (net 6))
 (segment (start 159.850666 97.62) (end 156.722 97.62) (width 0.8) (layer F.Cu) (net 6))
 (segment (start 156.722 97.62) (end 156.718 97.616) (width 0.8) (layer F.Cu) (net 6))
 (segment (start 171.449999 97.62) (end 170.247918 97.62) (width 0.8) (layer F.Cu) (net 6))
 (segment (start 170.247918 97.62) (end 159.850666 97.62) (width 0.8) (layer F.Cu) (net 6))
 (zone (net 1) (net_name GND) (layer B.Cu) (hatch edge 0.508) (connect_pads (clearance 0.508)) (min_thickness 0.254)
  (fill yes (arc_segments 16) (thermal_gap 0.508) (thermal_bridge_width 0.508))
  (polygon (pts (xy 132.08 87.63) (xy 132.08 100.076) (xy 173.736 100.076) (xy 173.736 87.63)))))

